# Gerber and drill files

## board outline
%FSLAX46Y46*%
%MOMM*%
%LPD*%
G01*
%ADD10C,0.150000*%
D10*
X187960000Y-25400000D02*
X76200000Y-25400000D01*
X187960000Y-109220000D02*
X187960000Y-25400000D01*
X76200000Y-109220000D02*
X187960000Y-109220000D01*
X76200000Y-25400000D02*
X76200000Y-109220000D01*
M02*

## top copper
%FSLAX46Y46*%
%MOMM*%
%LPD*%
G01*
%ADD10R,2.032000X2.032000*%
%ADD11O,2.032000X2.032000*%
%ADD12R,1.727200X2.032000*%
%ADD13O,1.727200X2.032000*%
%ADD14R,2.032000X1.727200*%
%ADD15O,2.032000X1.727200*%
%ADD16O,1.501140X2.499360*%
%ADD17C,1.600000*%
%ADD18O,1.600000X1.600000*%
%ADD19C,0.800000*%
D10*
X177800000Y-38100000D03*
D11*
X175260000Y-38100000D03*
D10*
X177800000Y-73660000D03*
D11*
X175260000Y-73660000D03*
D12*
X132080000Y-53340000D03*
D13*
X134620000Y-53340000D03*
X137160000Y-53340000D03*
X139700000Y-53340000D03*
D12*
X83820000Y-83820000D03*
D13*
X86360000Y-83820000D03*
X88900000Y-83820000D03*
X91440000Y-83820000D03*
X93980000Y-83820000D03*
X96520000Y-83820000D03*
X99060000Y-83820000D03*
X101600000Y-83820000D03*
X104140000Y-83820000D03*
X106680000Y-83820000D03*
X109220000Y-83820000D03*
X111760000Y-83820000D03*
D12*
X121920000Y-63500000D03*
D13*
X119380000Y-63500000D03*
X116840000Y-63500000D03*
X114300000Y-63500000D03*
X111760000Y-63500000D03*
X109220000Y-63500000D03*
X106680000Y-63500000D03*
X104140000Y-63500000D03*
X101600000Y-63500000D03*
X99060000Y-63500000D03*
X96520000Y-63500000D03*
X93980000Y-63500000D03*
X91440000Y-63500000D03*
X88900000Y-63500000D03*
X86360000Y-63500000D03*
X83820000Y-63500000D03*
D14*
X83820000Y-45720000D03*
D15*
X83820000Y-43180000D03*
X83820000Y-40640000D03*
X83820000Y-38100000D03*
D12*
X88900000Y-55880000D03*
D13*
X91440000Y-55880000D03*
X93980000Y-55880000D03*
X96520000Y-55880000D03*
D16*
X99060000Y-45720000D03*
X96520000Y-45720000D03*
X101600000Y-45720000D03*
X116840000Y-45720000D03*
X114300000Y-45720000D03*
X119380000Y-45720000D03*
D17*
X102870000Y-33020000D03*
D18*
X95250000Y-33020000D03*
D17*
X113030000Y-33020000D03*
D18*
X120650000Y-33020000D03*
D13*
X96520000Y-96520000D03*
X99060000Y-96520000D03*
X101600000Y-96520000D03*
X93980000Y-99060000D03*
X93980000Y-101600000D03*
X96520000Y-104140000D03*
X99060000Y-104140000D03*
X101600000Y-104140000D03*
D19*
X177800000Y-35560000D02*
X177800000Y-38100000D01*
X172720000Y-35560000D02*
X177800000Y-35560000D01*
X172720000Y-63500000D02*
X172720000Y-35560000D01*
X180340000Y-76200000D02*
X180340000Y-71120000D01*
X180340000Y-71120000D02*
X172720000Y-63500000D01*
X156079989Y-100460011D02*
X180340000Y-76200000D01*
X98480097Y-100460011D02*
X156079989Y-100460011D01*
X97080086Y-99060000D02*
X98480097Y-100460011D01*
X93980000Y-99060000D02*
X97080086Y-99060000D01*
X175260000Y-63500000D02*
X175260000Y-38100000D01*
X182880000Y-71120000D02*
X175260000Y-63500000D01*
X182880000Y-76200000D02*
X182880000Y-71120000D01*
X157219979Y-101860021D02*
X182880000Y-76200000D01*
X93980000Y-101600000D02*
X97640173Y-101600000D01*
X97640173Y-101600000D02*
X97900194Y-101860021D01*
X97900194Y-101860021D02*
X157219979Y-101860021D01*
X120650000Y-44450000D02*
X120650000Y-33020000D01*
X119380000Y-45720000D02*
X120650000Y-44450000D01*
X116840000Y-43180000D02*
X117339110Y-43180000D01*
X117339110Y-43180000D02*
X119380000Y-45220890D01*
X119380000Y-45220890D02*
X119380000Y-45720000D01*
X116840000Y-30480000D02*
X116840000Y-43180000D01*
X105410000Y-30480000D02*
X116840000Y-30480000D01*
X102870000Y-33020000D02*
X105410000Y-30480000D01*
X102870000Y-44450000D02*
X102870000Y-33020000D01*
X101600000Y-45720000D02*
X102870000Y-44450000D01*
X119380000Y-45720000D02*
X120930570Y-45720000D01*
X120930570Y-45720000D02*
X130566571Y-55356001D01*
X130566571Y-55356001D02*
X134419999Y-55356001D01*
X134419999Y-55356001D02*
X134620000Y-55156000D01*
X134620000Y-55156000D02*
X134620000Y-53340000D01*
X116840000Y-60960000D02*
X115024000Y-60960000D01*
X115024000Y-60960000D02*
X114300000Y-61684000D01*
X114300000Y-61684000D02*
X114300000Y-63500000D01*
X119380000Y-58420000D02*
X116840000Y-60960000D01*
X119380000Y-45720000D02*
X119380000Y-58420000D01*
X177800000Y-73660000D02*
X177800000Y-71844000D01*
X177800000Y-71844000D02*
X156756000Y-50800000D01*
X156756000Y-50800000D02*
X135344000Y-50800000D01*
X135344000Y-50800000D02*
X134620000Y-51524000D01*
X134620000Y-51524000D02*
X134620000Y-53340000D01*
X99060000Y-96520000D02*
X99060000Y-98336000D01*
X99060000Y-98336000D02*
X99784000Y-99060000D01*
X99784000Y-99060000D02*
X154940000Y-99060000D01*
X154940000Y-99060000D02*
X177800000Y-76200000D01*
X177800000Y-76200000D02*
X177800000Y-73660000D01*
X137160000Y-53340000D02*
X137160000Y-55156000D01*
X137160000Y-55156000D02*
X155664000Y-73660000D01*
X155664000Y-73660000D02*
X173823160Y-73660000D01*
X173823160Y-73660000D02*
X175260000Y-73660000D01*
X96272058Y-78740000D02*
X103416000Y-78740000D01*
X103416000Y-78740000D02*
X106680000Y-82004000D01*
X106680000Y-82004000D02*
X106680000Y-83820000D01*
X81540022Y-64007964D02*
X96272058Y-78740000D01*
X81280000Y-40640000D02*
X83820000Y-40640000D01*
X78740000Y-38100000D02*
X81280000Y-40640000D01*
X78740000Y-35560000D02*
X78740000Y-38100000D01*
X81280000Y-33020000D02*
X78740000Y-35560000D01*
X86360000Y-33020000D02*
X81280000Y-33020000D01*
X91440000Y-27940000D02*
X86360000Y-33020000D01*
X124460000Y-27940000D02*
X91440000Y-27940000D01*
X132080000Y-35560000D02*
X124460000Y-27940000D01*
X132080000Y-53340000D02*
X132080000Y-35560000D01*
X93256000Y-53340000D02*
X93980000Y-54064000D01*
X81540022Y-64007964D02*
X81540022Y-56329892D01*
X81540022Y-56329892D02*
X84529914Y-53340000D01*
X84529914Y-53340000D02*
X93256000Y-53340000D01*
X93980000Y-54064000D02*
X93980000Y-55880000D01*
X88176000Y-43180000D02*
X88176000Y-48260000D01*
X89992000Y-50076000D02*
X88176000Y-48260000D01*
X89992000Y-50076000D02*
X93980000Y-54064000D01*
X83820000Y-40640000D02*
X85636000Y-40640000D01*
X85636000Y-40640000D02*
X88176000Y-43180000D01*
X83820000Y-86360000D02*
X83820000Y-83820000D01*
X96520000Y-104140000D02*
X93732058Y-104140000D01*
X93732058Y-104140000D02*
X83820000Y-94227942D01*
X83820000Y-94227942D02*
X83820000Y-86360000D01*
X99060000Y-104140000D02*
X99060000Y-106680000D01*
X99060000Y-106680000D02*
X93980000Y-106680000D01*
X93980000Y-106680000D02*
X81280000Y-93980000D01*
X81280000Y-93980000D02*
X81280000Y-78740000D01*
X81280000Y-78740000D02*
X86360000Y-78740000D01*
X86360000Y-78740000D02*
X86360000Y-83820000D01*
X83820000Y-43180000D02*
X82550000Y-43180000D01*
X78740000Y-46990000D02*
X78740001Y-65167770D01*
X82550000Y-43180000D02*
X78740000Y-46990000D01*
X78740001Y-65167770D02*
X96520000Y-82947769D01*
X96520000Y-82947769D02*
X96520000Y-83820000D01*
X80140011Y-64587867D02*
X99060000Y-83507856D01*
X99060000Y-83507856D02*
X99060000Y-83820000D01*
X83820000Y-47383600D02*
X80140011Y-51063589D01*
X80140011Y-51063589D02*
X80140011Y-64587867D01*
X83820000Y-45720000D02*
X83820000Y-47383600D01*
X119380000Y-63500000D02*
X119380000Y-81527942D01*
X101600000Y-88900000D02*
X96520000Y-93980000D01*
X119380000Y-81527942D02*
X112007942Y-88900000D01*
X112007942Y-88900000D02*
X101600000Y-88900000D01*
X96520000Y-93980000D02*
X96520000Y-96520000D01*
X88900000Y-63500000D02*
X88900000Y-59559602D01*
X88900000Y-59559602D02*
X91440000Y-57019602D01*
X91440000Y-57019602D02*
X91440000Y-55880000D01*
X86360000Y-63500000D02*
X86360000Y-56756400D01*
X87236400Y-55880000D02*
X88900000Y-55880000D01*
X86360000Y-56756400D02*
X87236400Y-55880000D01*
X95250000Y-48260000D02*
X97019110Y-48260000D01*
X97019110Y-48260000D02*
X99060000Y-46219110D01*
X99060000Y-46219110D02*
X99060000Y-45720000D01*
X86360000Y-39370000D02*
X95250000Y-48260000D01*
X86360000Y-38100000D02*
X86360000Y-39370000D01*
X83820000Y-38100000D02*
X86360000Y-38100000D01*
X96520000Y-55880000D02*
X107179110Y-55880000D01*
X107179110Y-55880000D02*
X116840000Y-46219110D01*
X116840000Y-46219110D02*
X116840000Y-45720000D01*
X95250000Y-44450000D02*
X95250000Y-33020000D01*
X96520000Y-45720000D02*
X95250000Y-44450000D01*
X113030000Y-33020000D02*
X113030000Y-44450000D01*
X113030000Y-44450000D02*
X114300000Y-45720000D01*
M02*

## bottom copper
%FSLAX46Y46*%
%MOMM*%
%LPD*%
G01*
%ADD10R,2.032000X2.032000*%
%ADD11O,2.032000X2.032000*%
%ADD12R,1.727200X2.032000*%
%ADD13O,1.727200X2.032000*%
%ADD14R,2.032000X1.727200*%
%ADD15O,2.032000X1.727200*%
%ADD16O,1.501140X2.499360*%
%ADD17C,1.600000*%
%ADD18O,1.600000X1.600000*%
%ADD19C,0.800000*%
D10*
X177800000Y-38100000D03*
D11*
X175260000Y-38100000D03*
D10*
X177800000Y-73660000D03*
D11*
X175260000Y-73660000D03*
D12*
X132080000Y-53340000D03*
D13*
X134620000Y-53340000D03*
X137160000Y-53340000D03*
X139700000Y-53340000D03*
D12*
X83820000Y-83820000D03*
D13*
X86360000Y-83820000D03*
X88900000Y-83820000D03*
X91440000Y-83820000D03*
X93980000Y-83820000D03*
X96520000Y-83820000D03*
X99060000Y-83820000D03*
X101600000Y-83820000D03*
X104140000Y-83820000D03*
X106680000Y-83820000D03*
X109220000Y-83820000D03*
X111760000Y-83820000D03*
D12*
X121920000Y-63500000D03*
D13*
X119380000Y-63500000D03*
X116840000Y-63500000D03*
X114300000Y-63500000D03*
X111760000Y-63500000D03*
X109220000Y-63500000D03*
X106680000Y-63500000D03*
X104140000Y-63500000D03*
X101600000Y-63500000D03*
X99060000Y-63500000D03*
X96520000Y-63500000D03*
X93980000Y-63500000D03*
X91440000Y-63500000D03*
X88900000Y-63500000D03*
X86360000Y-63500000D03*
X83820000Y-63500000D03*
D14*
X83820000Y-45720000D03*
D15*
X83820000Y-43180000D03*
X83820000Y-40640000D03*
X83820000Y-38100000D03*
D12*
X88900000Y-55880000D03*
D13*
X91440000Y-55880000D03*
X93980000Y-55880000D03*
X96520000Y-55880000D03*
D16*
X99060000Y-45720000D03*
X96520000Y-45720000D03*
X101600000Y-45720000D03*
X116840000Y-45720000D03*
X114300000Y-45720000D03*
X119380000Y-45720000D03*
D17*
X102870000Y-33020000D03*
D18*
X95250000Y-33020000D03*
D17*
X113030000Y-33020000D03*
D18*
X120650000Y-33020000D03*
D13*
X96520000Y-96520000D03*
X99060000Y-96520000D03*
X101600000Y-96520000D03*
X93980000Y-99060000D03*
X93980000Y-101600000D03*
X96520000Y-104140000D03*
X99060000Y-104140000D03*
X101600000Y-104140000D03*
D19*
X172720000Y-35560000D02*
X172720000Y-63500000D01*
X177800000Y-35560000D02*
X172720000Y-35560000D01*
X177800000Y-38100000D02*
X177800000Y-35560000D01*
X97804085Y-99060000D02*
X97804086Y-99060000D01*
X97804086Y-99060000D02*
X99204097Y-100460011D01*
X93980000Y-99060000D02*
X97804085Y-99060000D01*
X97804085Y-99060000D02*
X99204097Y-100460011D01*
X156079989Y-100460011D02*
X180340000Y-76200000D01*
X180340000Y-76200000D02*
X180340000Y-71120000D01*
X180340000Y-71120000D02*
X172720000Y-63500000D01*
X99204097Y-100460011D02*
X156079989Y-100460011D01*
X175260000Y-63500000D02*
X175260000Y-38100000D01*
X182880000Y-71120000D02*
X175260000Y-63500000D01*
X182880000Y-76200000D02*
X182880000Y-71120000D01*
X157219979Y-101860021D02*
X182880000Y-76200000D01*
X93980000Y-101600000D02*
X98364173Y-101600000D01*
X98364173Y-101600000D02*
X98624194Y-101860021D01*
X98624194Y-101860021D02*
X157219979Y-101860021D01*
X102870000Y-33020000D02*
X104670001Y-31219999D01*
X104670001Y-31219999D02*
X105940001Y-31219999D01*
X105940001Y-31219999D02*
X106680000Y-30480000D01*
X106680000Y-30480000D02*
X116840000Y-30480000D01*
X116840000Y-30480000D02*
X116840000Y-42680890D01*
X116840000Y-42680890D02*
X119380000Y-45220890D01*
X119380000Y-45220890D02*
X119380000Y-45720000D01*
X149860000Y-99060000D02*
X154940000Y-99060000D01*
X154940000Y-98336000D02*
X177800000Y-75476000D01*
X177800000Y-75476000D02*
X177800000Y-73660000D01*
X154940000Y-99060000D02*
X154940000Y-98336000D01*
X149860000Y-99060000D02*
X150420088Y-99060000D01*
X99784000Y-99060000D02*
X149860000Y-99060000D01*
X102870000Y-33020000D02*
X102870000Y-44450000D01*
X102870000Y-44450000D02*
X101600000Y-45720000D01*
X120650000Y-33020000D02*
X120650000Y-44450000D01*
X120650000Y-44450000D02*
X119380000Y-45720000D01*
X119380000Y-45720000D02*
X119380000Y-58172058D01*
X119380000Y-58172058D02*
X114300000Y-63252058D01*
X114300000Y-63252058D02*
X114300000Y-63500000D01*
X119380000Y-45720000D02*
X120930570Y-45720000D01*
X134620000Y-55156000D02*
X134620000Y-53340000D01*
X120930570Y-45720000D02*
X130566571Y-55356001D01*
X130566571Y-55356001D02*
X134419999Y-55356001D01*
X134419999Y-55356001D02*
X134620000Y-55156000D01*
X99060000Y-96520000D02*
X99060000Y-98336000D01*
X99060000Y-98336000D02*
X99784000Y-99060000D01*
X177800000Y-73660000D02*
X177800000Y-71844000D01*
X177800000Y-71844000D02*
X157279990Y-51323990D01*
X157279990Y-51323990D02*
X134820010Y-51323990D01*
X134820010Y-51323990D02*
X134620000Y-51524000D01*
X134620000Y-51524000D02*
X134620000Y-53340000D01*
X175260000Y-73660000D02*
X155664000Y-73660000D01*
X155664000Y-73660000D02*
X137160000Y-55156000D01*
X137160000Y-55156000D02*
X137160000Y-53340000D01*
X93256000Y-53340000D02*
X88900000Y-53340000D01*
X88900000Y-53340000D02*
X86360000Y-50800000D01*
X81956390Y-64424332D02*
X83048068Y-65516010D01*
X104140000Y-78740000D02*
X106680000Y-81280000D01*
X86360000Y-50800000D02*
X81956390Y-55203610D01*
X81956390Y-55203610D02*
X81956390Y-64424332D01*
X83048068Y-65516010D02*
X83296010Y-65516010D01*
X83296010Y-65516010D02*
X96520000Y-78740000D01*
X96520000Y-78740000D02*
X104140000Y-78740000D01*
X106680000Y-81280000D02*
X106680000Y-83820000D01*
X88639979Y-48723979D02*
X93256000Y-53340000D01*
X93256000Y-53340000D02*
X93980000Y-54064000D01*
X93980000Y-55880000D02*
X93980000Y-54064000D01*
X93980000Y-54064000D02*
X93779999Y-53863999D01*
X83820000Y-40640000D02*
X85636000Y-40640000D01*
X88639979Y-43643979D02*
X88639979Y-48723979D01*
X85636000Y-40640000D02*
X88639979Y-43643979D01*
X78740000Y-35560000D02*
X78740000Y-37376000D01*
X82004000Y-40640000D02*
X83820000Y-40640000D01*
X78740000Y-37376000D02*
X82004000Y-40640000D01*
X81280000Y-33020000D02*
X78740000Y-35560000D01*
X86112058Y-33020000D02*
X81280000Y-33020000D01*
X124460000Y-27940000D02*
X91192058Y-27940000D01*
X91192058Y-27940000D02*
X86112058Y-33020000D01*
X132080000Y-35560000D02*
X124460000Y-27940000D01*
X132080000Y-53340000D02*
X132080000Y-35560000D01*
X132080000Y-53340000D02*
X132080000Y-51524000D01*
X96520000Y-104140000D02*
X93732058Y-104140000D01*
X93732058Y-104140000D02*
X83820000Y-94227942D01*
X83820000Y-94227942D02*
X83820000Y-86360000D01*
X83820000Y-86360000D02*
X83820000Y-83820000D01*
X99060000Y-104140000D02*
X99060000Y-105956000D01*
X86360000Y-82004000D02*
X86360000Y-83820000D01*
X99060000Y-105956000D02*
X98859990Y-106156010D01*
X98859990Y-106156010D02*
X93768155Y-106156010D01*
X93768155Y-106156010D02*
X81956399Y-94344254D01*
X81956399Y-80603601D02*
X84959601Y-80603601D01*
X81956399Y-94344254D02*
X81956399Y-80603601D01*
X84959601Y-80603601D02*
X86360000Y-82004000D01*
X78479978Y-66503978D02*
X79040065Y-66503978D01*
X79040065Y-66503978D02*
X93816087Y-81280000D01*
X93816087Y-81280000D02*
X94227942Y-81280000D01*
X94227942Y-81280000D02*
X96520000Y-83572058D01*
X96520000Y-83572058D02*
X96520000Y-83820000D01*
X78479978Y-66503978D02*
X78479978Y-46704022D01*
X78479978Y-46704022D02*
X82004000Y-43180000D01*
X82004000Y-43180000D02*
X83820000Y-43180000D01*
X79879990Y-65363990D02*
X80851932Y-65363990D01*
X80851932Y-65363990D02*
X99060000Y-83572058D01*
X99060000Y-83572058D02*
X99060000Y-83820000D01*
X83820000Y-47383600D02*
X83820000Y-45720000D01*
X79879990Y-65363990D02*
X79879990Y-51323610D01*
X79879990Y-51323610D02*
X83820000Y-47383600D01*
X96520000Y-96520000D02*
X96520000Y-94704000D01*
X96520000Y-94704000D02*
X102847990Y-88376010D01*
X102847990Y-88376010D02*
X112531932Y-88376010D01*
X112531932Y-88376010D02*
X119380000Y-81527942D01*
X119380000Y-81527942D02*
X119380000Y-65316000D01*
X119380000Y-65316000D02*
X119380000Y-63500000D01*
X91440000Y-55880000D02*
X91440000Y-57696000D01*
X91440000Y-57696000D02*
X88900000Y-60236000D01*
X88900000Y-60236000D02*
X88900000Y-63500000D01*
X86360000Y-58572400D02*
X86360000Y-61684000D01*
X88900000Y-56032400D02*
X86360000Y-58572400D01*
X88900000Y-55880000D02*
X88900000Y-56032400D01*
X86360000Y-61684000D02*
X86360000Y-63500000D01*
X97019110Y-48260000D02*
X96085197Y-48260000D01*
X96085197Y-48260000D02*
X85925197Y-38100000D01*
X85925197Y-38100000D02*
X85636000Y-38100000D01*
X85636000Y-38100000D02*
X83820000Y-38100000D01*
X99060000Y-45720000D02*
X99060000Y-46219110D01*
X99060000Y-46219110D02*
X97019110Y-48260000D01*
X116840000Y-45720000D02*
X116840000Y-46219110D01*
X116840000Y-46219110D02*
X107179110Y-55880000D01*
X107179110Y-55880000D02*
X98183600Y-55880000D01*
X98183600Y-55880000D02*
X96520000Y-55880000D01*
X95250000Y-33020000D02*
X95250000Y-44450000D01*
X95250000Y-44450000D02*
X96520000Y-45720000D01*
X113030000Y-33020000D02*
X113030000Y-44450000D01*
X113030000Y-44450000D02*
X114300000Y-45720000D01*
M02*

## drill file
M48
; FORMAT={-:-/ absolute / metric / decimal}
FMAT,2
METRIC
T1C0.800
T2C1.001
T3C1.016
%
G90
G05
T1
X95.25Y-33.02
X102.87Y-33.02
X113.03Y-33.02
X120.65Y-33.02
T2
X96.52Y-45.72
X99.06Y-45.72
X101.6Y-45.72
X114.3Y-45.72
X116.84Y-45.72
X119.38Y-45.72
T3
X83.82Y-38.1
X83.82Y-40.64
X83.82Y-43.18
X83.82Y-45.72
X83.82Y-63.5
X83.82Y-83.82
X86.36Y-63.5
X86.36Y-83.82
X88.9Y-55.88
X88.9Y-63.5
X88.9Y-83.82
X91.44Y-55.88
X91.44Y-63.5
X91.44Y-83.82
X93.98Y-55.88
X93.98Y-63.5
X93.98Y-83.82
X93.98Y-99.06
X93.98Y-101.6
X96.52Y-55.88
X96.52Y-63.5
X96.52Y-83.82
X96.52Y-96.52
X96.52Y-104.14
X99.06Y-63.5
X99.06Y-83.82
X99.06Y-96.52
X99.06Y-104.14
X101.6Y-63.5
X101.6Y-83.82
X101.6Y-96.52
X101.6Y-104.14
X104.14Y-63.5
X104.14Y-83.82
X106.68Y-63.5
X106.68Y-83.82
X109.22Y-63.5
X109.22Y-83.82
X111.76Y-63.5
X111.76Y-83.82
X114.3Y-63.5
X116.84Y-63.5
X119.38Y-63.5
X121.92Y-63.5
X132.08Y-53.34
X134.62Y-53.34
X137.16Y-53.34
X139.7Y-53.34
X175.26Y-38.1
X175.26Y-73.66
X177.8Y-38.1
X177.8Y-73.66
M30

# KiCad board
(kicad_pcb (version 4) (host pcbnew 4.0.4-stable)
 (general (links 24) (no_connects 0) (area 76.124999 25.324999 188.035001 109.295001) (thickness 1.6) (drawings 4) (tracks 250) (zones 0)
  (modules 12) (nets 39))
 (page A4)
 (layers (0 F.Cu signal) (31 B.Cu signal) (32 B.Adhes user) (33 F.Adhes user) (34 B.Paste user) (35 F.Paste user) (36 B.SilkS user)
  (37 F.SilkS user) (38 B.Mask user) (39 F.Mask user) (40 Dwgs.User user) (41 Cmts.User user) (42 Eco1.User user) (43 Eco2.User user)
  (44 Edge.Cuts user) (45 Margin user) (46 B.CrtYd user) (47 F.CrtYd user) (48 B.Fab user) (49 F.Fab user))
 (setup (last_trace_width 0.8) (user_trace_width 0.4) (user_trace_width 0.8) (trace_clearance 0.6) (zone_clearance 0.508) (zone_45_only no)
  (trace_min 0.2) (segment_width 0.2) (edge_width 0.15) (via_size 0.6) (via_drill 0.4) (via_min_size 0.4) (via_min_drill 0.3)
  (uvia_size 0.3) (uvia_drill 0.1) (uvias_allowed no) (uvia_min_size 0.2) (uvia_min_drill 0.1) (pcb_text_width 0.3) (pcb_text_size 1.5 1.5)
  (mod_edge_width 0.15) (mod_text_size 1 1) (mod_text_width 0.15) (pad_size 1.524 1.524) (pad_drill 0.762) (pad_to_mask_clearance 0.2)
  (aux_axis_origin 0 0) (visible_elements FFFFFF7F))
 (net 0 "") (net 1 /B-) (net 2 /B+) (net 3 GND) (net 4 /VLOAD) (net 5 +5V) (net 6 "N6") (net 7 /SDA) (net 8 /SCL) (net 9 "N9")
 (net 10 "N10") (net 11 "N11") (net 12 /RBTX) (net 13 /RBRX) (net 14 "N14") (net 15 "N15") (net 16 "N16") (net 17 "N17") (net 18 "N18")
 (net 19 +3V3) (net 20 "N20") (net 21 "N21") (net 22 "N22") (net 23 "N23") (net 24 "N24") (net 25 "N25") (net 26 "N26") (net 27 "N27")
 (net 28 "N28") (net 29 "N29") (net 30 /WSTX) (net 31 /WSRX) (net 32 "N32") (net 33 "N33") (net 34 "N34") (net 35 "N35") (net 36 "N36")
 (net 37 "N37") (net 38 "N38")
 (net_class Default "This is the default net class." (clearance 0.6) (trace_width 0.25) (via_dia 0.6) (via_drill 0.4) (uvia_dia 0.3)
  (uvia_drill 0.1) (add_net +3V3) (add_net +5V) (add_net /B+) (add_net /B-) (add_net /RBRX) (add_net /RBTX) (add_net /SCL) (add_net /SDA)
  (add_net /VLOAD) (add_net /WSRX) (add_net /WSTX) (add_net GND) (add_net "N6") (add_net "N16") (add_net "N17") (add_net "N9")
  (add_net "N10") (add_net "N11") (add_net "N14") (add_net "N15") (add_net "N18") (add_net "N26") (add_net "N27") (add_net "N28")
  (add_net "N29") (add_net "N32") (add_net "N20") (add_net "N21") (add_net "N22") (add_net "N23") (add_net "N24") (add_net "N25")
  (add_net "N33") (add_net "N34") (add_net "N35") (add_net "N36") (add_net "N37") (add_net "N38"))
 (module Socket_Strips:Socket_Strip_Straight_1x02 (layer F.Cu) (at 177.8 38.1 180)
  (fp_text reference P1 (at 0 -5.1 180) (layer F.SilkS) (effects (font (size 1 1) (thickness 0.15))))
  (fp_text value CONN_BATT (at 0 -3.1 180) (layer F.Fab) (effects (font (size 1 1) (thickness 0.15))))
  (pad 1 thru_hole rect (at 0 0 180) (size 2.032 2.032) (drill 1.016) (layers *.Cu *.Mask) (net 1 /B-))
  (pad 2 thru_hole oval (at 2.54 0 180) (size 2.032 2.032) (drill 1.016) (layers *.Cu *.Mask) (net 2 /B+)))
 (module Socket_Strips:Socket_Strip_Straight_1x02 (layer F.Cu) (at 177.8 73.66 180)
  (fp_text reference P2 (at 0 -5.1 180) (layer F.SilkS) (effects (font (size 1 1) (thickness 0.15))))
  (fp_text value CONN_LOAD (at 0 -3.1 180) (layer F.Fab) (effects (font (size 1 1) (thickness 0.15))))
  (pad 1 thru_hole rect (at 0 0 180) (size 2.032 2.032) (drill 1.016) (layers *.Cu *.Mask) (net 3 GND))
  (pad 2 thru_hole oval (at 2.54 0 180) (size 2.032 2.032) (drill 1.016) (layers *.Cu *.Mask) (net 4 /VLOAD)))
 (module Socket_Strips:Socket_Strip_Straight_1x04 (layer F.Cu) (at 132.08 53.34)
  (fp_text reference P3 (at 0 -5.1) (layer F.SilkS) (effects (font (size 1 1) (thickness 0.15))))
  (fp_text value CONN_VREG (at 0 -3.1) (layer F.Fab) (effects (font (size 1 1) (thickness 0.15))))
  (pad 1 thru_hole rect (at 0 0) (size 1.7272 2.032) (drill 1.016) (layers *.Cu *.Mask) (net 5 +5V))
  (pad 2 thru_hole oval (at 2.54 0) (size 1.7272 2.032) (drill 1.016) (layers *.Cu *.Mask) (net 3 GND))
  (pad 3 thru_hole oval (at 5.08 0) (size 1.7272 2.032) (drill 1.016) (layers *.Cu *.Mask) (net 4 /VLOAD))
  (pad 4 thru_hole oval (at 7.62 0) (size 1.7272 2.032) (drill 1.016) (layers *.Cu *.Mask) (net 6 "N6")))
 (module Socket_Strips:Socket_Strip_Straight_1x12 (layer F.Cu) (at 83.82 83.82)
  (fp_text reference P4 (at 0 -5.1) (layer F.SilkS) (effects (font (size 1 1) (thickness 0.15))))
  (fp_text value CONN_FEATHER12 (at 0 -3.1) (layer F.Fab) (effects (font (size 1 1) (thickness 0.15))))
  (pad 1 thru_hole rect (at 0 0) (size 1.7272 2.032) (drill 1.016) (layers *.Cu *.Mask) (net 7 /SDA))
  (pad 2 thru_hole oval (at 2.54 0) (size 1.7272 2.032) (drill 1.016) (layers *.Cu *.Mask) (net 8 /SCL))
  (pad 3 thru_hole oval (at 5.08 0) (size 1.7272 2.032) (drill 1.016) (layers *.Cu *.Mask) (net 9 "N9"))
  (pad 4 thru_hole oval (at 7.62 0) (size 1.7272 2.032) (drill 1.016) (layers *.Cu *.Mask) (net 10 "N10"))
  (pad 5 thru_hole oval (at 10.16 0) (size 1.7272 2.032) (drill 1.016) (layers *.Cu *.Mask) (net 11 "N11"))
  (pad 6 thru_hole oval (at 12.7 0) (size 1.7272 2.032) (drill 1.016) (layers *.Cu *.Mask) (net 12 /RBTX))
  (pad 7 thru_hole oval (at 15.24 0) (size 1.7272 2.032) (drill 1.016) (layers *.Cu *.Mask) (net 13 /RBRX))
  (pad 8 thru_hole oval (at 17.78 0) (size 1.7272 2.032) (drill 1.016) (layers *.Cu *.Mask) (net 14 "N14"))
  (pad 9 thru_hole oval (at 20.32 0) (size 1.7272 2.032) (drill 1.016) (layers *.Cu *.Mask) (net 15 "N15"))
  (pad 10 thru_hole oval (at 22.86 0) (size 1.7272 2.032) (drill 1.016) (layers *.Cu *.Mask) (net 5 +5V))
  (pad 11 thru_hole oval (at 25.4 0) (size 1.7272 2.032) (drill 1.016) (layers *.Cu *.Mask) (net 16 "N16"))
  (pad 12 thru_hole oval (at 27.94 0) (size 1.7272 2.032) (drill 1.016) (layers *.Cu *.Mask) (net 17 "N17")))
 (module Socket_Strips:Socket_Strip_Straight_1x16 (layer F.Cu) (at 121.92 63.5 180)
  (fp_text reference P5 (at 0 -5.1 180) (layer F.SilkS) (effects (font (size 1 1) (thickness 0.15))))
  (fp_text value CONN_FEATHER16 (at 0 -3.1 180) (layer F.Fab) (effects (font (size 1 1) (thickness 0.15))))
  (pad 1 thru_hole rect (at 0 0 180) (size 1.7272 2.032) (drill 1.016) (layers *.Cu *.Mask) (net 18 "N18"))
  (pad 2 thru_hole oval (at 2.54 0 180) (size 1.7272 2.032) (drill 1.016) (layers *.Cu *.Mask) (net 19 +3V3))
  (pad 3 thru_hole oval (at 5.08 0 180) (size 1.7272 2.032) (drill 1.016) (layers *.Cu *.Mask) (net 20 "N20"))
  (pad 4 thru_hole oval (at 7.62 0 180) (size 1.7272 2.032) (drill 1.016) (layers *.Cu *.Mask) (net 3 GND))
  (pad 5 thru_hole oval (at 10.16 0 180) (size 1.7272 2.032) (drill 1.016) (layers *.Cu *.Mask) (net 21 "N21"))
  (pad 6 thru_hole oval (at 12.7 0 180) (size 1.7272 2.032) (drill 1.016) (layers *.Cu *.Mask) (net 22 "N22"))
  (pad 7 thru_hole oval (at 15.24 0 180) (size 1.7272 2.032) (drill 1.016) (layers *.Cu *.Mask) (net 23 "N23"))
  (pad 8 thru_hole oval (at 17.78 0 180) (size 1.7272 2.032) (drill 1.016) (layers *.Cu *.Mask) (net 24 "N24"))
  (pad 9 thru_hole oval (at 20.32 0 180) (size 1.7272 2.032) (drill 1.016) (layers *.Cu *.Mask) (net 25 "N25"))
  (pad 10 thru_hole oval (at 22.86 0 180) (size 1.7272 2.032) (drill 1.016) (layers *.Cu *.Mask) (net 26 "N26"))
  (pad 11 thru_hole oval (at 25.4 0 180) (size 1.7272 2.032) (drill 1.016) (layers *.Cu *.Mask) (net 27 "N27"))
  (pad 12 thru_hole oval (at 27.94 0 180) (size 1.7272 2.032) (drill 1.016) (layers *.Cu *.Mask) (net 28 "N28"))
  (pad 13 thru_hole oval (at 30.48 0 180) (size 1.7272 2.032) (drill 1.016) (layers *.Cu *.Mask) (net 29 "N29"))
  (pad 14 thru_hole oval (at 33.02 0 180) (size 1.7272 2.032) (drill 1.016) (layers *.Cu *.Mask) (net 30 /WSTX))
  (pad 15 thru_hole oval (at 35.56 0 180) (size 1.7272 2.032) (drill 1.016) (layers *.Cu *.Mask) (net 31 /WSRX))
  (pad 16 thru_hole oval (at 38.1 0 180) (size 1.7272 2.032) (drill 1.016) (layers *.Cu *.Mask) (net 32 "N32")))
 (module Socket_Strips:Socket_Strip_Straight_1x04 (layer F.Cu) (at 83.82 45.72 90)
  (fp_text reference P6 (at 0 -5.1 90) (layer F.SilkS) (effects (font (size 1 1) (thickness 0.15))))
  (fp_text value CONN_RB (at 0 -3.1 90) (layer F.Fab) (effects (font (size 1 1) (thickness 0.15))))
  (pad 1 thru_hole rect (at 0 0 90) (size 1.7272 2.032) (drill 1.016) (layers *.Cu *.Mask) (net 13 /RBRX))
  (pad 2 thru_hole oval (at 2.54 0 90) (size 1.7272 2.032) (drill 1.016) (layers *.Cu *.Mask) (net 12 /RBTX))
  (pad 3 thru_hole oval (at 5.08 0 90) (size 1.7272 2.032) (drill 1.016) (layers *.Cu *.Mask) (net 5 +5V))
  (pad 4 thru_hole oval (at 7.62 0 90) (size 1.7272 2.032) (drill 1.016) (layers *.Cu *.Mask) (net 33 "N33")))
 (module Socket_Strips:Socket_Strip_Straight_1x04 (layer F.Cu) (at 88.9 55.88)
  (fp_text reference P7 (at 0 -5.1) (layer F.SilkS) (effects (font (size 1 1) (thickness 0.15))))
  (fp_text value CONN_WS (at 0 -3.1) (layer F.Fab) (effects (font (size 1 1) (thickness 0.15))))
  (pad 1 thru_hole rect (at 0 0) (size 1.7272 2.032) (drill 1.016) (layers *.Cu *.Mask) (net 31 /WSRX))
  (pad 2 thru_hole oval (at 2.54 0) (size 1.7272 2.032) (drill 1.016) (layers *.Cu *.Mask) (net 30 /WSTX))
  (pad 3 thru_hole oval (at 5.08 0) (size 1.7272 2.032) (drill 1.016) (layers *.Cu *.Mask) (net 5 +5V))
  (pad 4 thru_hole oval (at 7.62 0) (size 1.7272 2.032) (drill 1.016) (layers *.Cu *.Mask) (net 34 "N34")))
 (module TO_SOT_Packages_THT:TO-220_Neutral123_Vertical (layer F.Cu) (at 99.06 45.72)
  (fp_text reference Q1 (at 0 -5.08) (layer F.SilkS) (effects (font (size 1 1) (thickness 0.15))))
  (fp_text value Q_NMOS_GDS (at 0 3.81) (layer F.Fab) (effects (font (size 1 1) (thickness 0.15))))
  (pad 2 thru_hole oval (at 0 0 90) (size 2.49936 1.50114) (drill 1.00076) (layers *.Cu *.Mask) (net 33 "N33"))
  (pad 1 thru_hole oval (at -2.54 0 90) (size 2.49936 1.50114) (drill 1.00076) (layers *.Cu *.Mask) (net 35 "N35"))
  (pad 3 thru_hole oval (at 2.54 0 90) (size 2.49936 1.50114) (drill 1.00076) (layers *.Cu *.Mask) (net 3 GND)))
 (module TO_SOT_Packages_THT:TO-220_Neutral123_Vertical (layer F.Cu) (at 116.84 45.72)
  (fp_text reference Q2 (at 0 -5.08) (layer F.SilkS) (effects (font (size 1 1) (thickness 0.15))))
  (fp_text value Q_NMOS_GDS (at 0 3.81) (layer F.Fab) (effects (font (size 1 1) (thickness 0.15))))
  (pad 2 thru_hole oval (at 0 0 90) (size 2.49936 1.50114) (drill 1.00076) (layers *.Cu *.Mask) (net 34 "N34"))
  (pad 1 thru_hole oval (at -2.54 0 90) (size 2.49936 1.50114) (drill 1.00076) (layers *.Cu *.Mask) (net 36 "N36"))
  (pad 3 thru_hole oval (at 2.54 0 90) (size 2.49936 1.50114) (drill 1.00076) (layers *.Cu *.Mask) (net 3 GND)))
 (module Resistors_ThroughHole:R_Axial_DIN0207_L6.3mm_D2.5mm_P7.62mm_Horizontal (layer F.Cu) (at 102.87 33.02 180)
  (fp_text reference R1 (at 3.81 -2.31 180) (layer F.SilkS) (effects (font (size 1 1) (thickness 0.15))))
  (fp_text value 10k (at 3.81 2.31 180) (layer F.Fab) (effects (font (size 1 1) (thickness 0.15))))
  (pad 1 thru_hole circle (at 0 0 180) (size 1.6 1.6) (drill 0.8) (layers *.Cu *.Mask) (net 3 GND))
  (pad 2 thru_hole oval (at 7.62 0 180) (size 1.6 1.6) (drill 0.8) (layers *.Cu *.Mask) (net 35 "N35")))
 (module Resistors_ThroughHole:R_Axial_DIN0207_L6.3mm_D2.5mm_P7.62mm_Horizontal (layer F.Cu) (at 113.03 33.02)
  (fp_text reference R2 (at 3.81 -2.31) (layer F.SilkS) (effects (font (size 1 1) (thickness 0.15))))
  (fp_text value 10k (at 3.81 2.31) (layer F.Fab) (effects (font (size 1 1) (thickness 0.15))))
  (pad 1 thru_hole circle (at 0 0) (size 1.6 1.6) (drill 0.8) (layers *.Cu *.Mask) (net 36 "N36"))
  (pad 2 thru_hole oval (at 7.62 0) (size 1.6 1.6) (drill 0.8) (layers *.Cu *.Mask) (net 3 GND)))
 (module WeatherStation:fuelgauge (layer F.Cu) (at 93.98 96.52)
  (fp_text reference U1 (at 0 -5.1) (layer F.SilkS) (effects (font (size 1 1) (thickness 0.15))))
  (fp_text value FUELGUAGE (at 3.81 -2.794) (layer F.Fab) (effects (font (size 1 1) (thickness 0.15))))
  (pad 3 thru_hole oval (at 2.54 0) (size 1.7272 2.032) (drill 1.016) (layers *.Cu *.Mask) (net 19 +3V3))
  (pad 4 thru_hole oval (at 5.08 0) (size 1.7272 2.032) (drill 1.016) (layers *.Cu *.Mask) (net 3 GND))
  (pad 5 thru_hole oval (at 7.62 0) (size 1.7272 2.032) (drill 1.016) (layers *.Cu *.Mask) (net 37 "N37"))
  (pad 2 thru_hole oval (at 0 2.54) (size 1.7272 2.032) (drill 1.016) (layers *.Cu *.Mask) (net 1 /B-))
  (pad 1 thru_hole oval (at 0 5.08) (size 1.7272 2.032) (drill 1.016) (layers *.Cu *.Mask) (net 2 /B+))
  (pad 8 thru_hole oval (at 2.54 7.62) (size 1.7272 2.032) (drill 1.016) (layers *.Cu *.Mask) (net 7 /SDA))
  (pad 7 thru_hole oval (at 5.08 7.62) (size 1.7272 2.032) (drill 1.016) (layers *.Cu *.Mask) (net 8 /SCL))
  (pad 6 thru_hole oval (at 7.62 7.62) (size 1.7272 2.032) (drill 1.016) (layers *.Cu *.Mask) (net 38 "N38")))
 (gr_line (start 187.96 25.4) (end 76.2 25.4) (angle 90) (layer Edge.Cuts) (width 0.15))
 (gr_line (start 187.96 109.22) (end 187.96 25.4) (angle 90) (layer Edge.Cuts) (width 0.15))
 (gr_line (start 76.2 109.22) (end 187.96 109.22) (angle 90) (layer Edge.Cuts) (width 0.15))
 (gr_line (start 76.2 25.4) (end 76.2 109.22) (angle 90) (layer Edge.Cuts) (width 0.15))
 (segment (start 172.72 35.56) (end 172.72 63.5) (width 0.8) (layer B.Cu) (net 1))
 (segment (start 177.8 35.56) (end 172.72 35.56) (width 0.8) (layer B.Cu) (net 1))
 (segment (start 177.8 38.1) (end 177.8 35.56) (width 0.8) (layer B.Cu) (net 1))
 (segment (start 177.8 35.56) (end 177.8 38.1) (width 0.8) (layer F.Cu) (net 1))
 (segment (start 172.72 35.56) (end 177.8 35.56) (width 0.8) (layer F.Cu) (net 1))
 (segment (start 172.72 63.5) (end 172.72 35.56) (width 0.8) (layer F.Cu) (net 1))
 (segment (start 180.34 76.2) (end 180.34 71.12) (width 0.8) (layer F.Cu) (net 1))
 (segment (start 180.34 71.12) (end 172.72 63.5) (width 0.8) (layer F.Cu) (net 1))
 (segment (start 156.079989 100.460011) (end 180.34 76.2) (width 0.8) (layer F.Cu) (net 1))
 (segment (start 98.480097 100.460011) (end 156.079989 100.460011) (width 0.8) (layer F.Cu) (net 1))
 (segment (start 97.080086 99.06) (end 98.480097 100.460011) (width 0.8) (layer F.Cu) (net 1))
 (segment (start 93.98 99.06) (end 97.080086 99.06) (width 0.8) (layer F.Cu) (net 1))
 (segment (start 97.804085 99.06) (end 97.804086 99.06) (width 0.8) (layer B.Cu) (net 1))
 (segment (start 97.804086 99.06) (end 99.204097 100.460011) (width 0.8) (layer B.Cu) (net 1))
 (segment (start 93.98 99.06) (end 97.804085 99.06) (width 0.8) (layer B.Cu) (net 1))
 (segment (start 97.804085 99.06) (end 99.204097 100.460011) (width 0.8) (layer B.Cu) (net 1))
 (segment (start 156.079989 100.460011) (end 180.34 76.2) (width 0.8) (layer B.Cu) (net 1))
 (segment (start 180.34 76.2) (end 180.34 71.12) (width 0.8) (layer B.Cu) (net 1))
 (segment (start 180.34 71.12) (end 172.72 63.5) (width 0.8) (layer B.Cu) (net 1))
 (segment (start 99.204097 100.460011) (end 156.079989 100.460011) (width 0.8) (layer B.Cu) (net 1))
 (segment (start 175.26 63.5) (end 175.26 38.1) (width 0.8) (layer B.Cu) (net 2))
 (segment (start 182.88 71.12) (end 175.26 63.5) (width 0.8) (layer B.Cu) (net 2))
 (segment (start 182.88 76.2) (end 182.88 71.12) (width 0.8) (layer B.Cu) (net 2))
 (segment (start 157.219979 101.860021) (end 182.88 76.2) (width 0.8) (layer B.Cu) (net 2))
 (segment (start 93.98 101.6) (end 98.364173 101.6) (width 0.8) (layer B.Cu) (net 2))
 (segment (start 98.364173 101.6) (end 98.624194 101.860021) (width 0.8) (layer B.Cu) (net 2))
 (segment (start 98.624194 101.860021) (end 157.219979 101.860021) (width 0.8) (layer B.Cu) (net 2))
 (segment (start 175.26 63.5) (end 175.26 38.1) (width 0.8) (layer F.Cu) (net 2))
 (segment (start 182.88 71.12) (end 175.26 63.5) (width 0.8) (layer F.Cu) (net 2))
 (segment (start 182.88 76.2) (end 182.88 71.12) (width 0.8) (layer F.Cu) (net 2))
 (segment (start 157.219979 101.860021) (end 182.88 76.2) (width 0.8) (layer F.Cu) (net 2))
 (segment (start 93.98 101.6) (end 97.640173 101.6) (width 0.8) (layer F.Cu) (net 2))
 (segment (start 97.640173 101.6) (end 97.900194 101.860021) (width 0.8) (layer F.Cu) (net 2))
 (segment (start 97.900194 101.860021) (end 157.219979 101.860021) (width 0.8) (layer F.Cu) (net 2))
 (segment (start 120.65 44.45) (end 120.65 33.02) (width 0.8) (layer F.Cu) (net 3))
 (segment (start 119.38 45.72) (end 120.65 44.45) (width 0.8) (layer F.Cu) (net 3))
 (segment (start 116.84 43.18) (end 117.33911 43.18) (width 0.8) (layer F.Cu) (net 3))
 (segment (start 117.33911 43.18) (end 119.38 45.22089) (width 0.8) (layer F.Cu) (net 3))
 (segment (start 119.38 45.22089) (end 119.38 45.72) (width 0.8) (layer F.Cu) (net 3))
 (segment (start 116.84 30.48) (end 116.84 43.18) (width 0.8) (layer F.Cu) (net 3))
 (segment (start 105.41 30.48) (end 116.84 30.48) (width 0.8) (layer F.Cu) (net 3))
 (segment (start 102.87 33.02) (end 105.41 30.48) (width 0.8) (layer F.Cu) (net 3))
 (segment (start 102.87 44.45) (end 102.87 33.02) (width 0.8) (layer F.Cu) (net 3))
 (segment (start 101.6 45.72) (end 102.87 44.45) (width 0.8) (layer F.Cu) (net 3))
 (segment (start 119.38 45.72) (end 120.93057 45.72) (width 0.8) (layer F.Cu) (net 3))
 (segment (start 120.93057 45.72) (end 130.566571 55.356001) (width 0.8) (layer F.Cu) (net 3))
 (segment (start 130.566571 55.356001) (end 134.419999 55.356001) (width 0.8) (layer F.Cu) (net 3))
 (segment (start 134.419999 55.356001) (end 134.62 55.156) (width 0.8) (layer F.Cu) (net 3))
 (segment (start 134.62 55.156) (end 134.62 53.34) (width 0.8) (layer F.Cu) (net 3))
 (segment (start 116.84 60.96) (end 115.024 60.96) (width 0.8) (layer F.Cu) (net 3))
 (segment (start 115.024 60.96) (end 114.3 61.684) (width 0.8) (layer F.Cu) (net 3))
 (segment (start 114.3 61.684) (end 114.3 63.5) (width 0.8) (layer F.Cu) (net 3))
 (segment (start 119.38 58.42) (end 116.84 60.96) (width 0.8) (layer F.Cu) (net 3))
 (segment (start 119.38 45.72) (end 119.38 58.42) (width 0.8) (layer F.Cu) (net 3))
 (segment (start 177.8 73.66) (end 177.8 71.844) (width 0.8) (layer F.Cu) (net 3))
 (segment (start 177.8 71.844) (end 156.756 50.8) (width 0.8) (layer F.Cu) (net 3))
 (segment (start 156.756 50.8) (end 135.344 50.8) (width 0.8) (layer F.Cu) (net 3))
 (segment (start 135.344 50.8) (end 134.62 51.524) (width 0.8) (layer F.Cu) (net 3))
 (segment (start 134.62 51.524) (end 134.62 53.34) (width 0.8) (layer F.Cu) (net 3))
 (segment (start 99.06 96.52) (end 99.06 98.336) (width 0.8) (layer F.Cu) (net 3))
 (segment (start 99.06 98.336) (end 99.784 99.06) (width 0.8) (layer F.Cu) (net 3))
 (segment (start 99.784 99.06) (end 154.94 99.06) (width 0.8) (layer F.Cu) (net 3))
 (segment (start 154.94 99.06) (end 177.8 76.2) (width 0.8) (layer F.Cu) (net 3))
 (segment (start 177.8 76.2) (end 177.8 73.66) (width 0.8) (layer F.Cu) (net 3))
 (segment (start 102.87 33.02) (end 104.670001 31.219999) (width 0.8) (layer B.Cu) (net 3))
 (segment (start 104.670001 31.219999) (end 105.940001 31.219999) (width 0.8) (layer B.Cu) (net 3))
 (segment (start 105.940001 31.219999) (end 106.68 30.48) (width 0.8) (layer B.Cu) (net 3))
 (segment (start 106.68 30.48) (end 116.84 30.48) (width 0.8) (layer B.Cu) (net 3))
 (segment (start 116.84 30.48) (end 116.84 42.68089) (width 0.8) (layer B.Cu) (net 3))
 (segment (start 116.84 42.68089) (end 119.38 45.22089) (width 0.8) (layer B.Cu) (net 3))
 (segment (start 119.38 45.22089) (end 119.38 45.72) (width 0.8) (layer B.Cu) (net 3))
 (segment (start 149.86 99.06) (end 154.94 99.06) (width 0.8) (layer B.Cu) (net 3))
 (segment (start 154.94 98.336) (end 177.8 75.476) (width 0.8) (layer B.Cu) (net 3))
 (segment (start 177.8 75.476) (end 177.8 73.66) (width 0.8) (layer B.Cu) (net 3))
 (segment (start 154.94 99.06) (end 154.94 98.336) (width 0.8) (layer B.Cu) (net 3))
 (segment (start 149.86 99.06) (end 150.420088 99.06) (width 0.8) (layer B.Cu) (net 3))
 (segment (start 99.784 99.06) (end 149.86 99.06) (width 0.8) (layer B.Cu) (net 3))
 (segment (start 102.87 33.02) (end 102.87 44.45) (width 0.8) (layer B.Cu) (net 3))
 (segment (start 102.87 44.45) (end 101.6 45.72) (width 0.8) (layer B.Cu) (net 3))
 (segment (start 120.65 33.02) (end 120.65 44.45) (width 0.8) (layer B.Cu) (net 3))
 (segment (start 120.65 44.45) (end 119.38 45.72) (width 0.8) (layer B.Cu) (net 3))
 (segment (start 119.38 45.72) (end 119.38 58.172058) (width 0.8) (layer B.Cu) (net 3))
 (segment (start 119.38 58.172058) (end 114.3 63.252058) (width 0.8) (layer B.Cu) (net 3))
 (segment (start 114.3 63.252058) (end 114.3 63.5) (width 0.8) (layer B.Cu) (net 3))
 (segment (start 119.38 45.72) (end 120.93057 45.72) (width 0.8) (layer B.Cu) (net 3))
 (segment (start 134.62 55.156) (end 134.62 53.34) (width 0.8) (layer B.Cu) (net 3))
 (segment (start 120.93057 45.72) (end 130.566571 55.356001) (width 0.8) (layer B.Cu) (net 3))
 (segment (start 130.566571 55.356001) (end 134.419999 55.356001) (width 0.8) (layer B.Cu) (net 3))
 (segment (start 134.419999 55.356001) (end 134.62 55.156) (width 0.8) (layer B.Cu) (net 3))
 (segment (start 99.06 96.52) (end 99.06 98.336) (width 0.8) (layer B.Cu) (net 3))
 (segment (start 99.06 98.336) (end 99.784 99.06) (width 0.8) (layer B.Cu) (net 3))
 (segment (start 177.8 73.66) (end 177.8 71.844) (width 0.8) (layer B.Cu) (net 3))
 (segment (start 177.8 71.844) (end 157.27999 51.32399) (width 0.8) (layer B.Cu) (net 3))
 (segment (start 157.27999 51.32399) (end 134.82001 51.32399) (width 0.8) (layer B.Cu) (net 3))
 (segment (start 134.82001 51.32399) (end 134.62 51.524) (width 0.8) (layer B.Cu) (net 3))
 (segment (start 134.62 51.524) (end 134.62 53.34) (width 0.8) (layer B.Cu) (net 3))
 (segment (start 137.16 53.34) (end 137.16 55.156) (width 0.8) (layer F.Cu) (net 4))
 (segment (start 137.16 55.156) (end 155.664 73.66) (width 0.8) (layer F.Cu) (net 4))
 (segment (start 155.664 73.66) (end 173.82316 73.66) (width 0.8) (layer F.Cu) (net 4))
 (segment (start 173.82316 73.66) (end 175.26 73.66) (width 0.8) (layer F.Cu) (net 4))
 (segment (start 175.26 73.66) (end 155.664 73.66) (width 0.8) (layer B.Cu) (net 4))
 (segment (start 155.664 73.66) (end 137.16 55.156) (width 0.8) (layer B.Cu) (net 4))
 (segment (start 137.16 55.156) (end 137.16 53.34) (width 0.8) (layer B.Cu) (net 4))
 (segment (start 93.256 53.34) (end 88.9 53.34) (width 0.8) (layer B.Cu) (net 5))
 (segment (start 88.9 53.34) (end 86.36 50.8) (width 0.8) (layer B.Cu) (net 5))
 (segment (start 81.95639 64.424332) (end 83.048068 65.51601) (width 0.8) (layer B.Cu) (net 5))
 (segment (start 104.14 78.74) (end 106.68 81.28) (width 0.8) (layer B.Cu) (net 5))
 (segment (start 86.36 50.8) (end 81.95639 55.20361) (width 0.8) (layer B.Cu) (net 5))
 (segment (start 81.95639 55.20361) (end 81.95639 64.424332) (width 0.8) (layer B.Cu) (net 5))
 (segment (start 83.048068 65.51601) (end 83.29601 65.51601) (width 0.8) (layer B.Cu) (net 5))
 (segment (start 83.29601 65.51601) (end 96.52 78.74) (width 0.8) (layer B.Cu) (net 5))
 (segment (start 96.52 78.74) (end 104.14 78.74) (width 0.8) (layer B.Cu) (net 5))
 (segment (start 106.68 81.28) (end 106.68 83.82) (width 0.8) (layer B.Cu) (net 5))
 (segment (start 96.272058 78.74) (end 103.416 78.74) (width 0.8) (layer F.Cu) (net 5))
 (segment (start 103.416 78.74) (end 106.68 82.004) (width 0.8) (layer F.Cu) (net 5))
 (segment (start 106.68 82.004) (end 106.68 83.82) (width 0.8) (layer F.Cu) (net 5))
 (segment (start 81.540022 64.007964) (end 96.272058 78.74) (width 0.8) (layer F.Cu) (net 5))
 (segment (start 81.28 40.64) (end 83.82 40.64) (width 0.8) (layer F.Cu) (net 5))
 (segment (start 78.74 38.1) (end 81.28 40.64) (width 0.8) (layer F.Cu) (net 5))
 (segment (start 78.74 35.56) (end 78.74 38.1) (width 0.8) (layer F.Cu) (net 5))
 (segment (start 81.28 33.02) (end 78.74 35.56) (width 0.8) (layer F.Cu) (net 5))
 (segment (start 86.36 33.02) (end 81.28 33.02) (width 0.8) (layer F.Cu) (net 5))
 (segment (start 91.44 27.94) (end 86.36 33.02) (width 0.8) (layer F.Cu) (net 5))
 (segment (start 124.46 27.94) (end 91.44 27.94) (width 0.8) (layer F.Cu) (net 5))
 (segment (start 132.08 35.56) (end 124.46 27.94) (width 0.8) (layer F.Cu) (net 5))
 (segment (start 132.08 53.34) (end 132.08 35.56) (width 0.8) (layer F.Cu) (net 5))
 (segment (start 93.256 53.34) (end 93.98 54.064) (width 0.8) (layer F.Cu) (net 5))
 (segment (start 81.540022 64.007964) (end 81.540022 56.329892) (width 0.8) (layer F.Cu) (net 5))
 (segment (start 81.540022 56.329892) (end 84.529914 53.34) (width 0.8) (layer F.Cu) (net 5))
 (segment (start 84.529914 53.34) (end 93.256 53.34) (width 0.8) (layer F.Cu) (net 5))
 (segment (start 93.98 54.064) (end 93.98 55.88) (width 0.8) (layer F.Cu) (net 5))
 (segment (start 88.176 43.18) (end 88.176 48.26) (width 0.8) (layer F.Cu) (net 5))
 (segment (start 89.992 50.076) (end 88.176 48.26) (width 0.8) (layer F.Cu) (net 5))
 (segment (start 89.992 50.076) (end 93.98 54.064) (width 0.8) (layer F.Cu) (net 5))
 (segment (start 83.82 40.64) (end 85.636 40.64) (width 0.8) (layer F.Cu) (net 5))
 (segment (start 85.636 40.64) (end 88.176 43.18) (width 0.8) (layer F.Cu) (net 5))
 (segment (start 88.639979 48.723979) (end 93.256 53.34) (width 0.8) (layer B.Cu) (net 5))
 (segment (start 93.256 53.34) (end 93.98 54.064) (width 0.8) (layer B.Cu) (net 5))
 (segment (start 93.98 55.88) (end 93.98 54.064) (width 0.8) (layer B.Cu) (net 5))
 (segment (start 93.98 54.064) (end 93.779999 53.863999) (width 0.8) (layer B.Cu) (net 5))
 (segment (start 83.82 40.64) (end 85.636 40.64) (width 0.8) (layer B.Cu) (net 5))
 (segment (start 88.639979 43.643979) (end 88.639979 48.723979) (width 0.8) (layer B.Cu) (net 5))
 (segment (start 85.636 40.64) (end 88.639979 43.643979) (width 0.8) (layer B.Cu) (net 5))
 (segment (start 78.74 35.56) (end 78.74 37.376) (width 0.8) (layer B.Cu) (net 5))
 (segment (start 82.004 40.64) (end 83.82 40.64) (width 0.8) (layer B.Cu) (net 5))
 (segment (start 78.74 37.376) (end 82.004 40.64) (width 0.8) (layer B.Cu) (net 5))
 (segment (start 81.28 33.02) (end 78.74 35.56) (width 0.8) (layer B.Cu) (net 5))
 (segment (start 86.112058 33.02) (end 81.28 33.02) (width 0.8) (layer B.Cu) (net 5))
 (segment (start 124.46 27.94) (end 91.192058 27.94) (width 0.8) (layer B.Cu) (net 5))
 (segment (start 91.192058 27.94) (end 86.112058 33.02) (width 0.8) (layer B.Cu) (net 5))
 (segment (start 132.08 35.56) (end 124.46 27.94) (width 0.8) (layer B.Cu) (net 5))
 (segment (start 132.08 53.34) (end 132.08 35.56) (width 0.8) (layer B.Cu) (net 5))
 (segment (start 132.08 53.34) (end 132.08 51.524) (width 0.8) (layer B.Cu) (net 5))
 (segment (start 96.52 104.14) (end 93.732058 104.14) (width 0.8) (layer B.Cu) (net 7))
 (segment (start 93.732058 104.14) (end 83.82 94.227942) (width 0.8) (layer B.Cu) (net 7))
 (segment (start 83.82 94.227942) (end 83.82 86.36) (width 0.8) (layer B.Cu) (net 7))
 (segment (start 83.82 86.36) (end 83.82 83.82) (width 0.8) (layer B.Cu) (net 7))
 (segment (start 83.82 86.36) (end 83.82 83.82) (width 0.8) (layer F.Cu) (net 7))
 (segment (start 96.52 104.14) (end 93.732058 104.14) (width 0.8) (layer F.Cu) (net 7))
 (segment (start 93.732058 104.14) (end 83.82 94.227942) (width 0.8) (layer F.Cu) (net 7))
 (segment (start 83.82 94.227942) (end 83.82 86.36) (width 0.8) (layer F.Cu) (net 7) (status 20))
 (segment (start 99.06 104.14) (end 99.06 105.956) (width 0.8) (layer B.Cu) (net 8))
 (segment (start 86.36 82.004) (end 86.36 83.82) (width 0.8) (layer B.Cu) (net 8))
 (segment (start 99.06 105.956) (end 98.85999 106.15601) (width 0.8) (layer B.Cu) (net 8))
 (segment (start 98.85999 106.15601) (end 93.768155 106.15601) (width 0.8) (layer B.Cu) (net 8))
 (segment (start 93.768155 106.15601) (end 81.956399 94.344254) (width 0.8) (layer B.Cu) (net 8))
 (segment (start 81.956399 80.603601) (end 84.959601 80.603601) (width 0.8) (layer B.Cu) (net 8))
 (segment (start 81.956399 94.344254) (end 81.956399 80.603601) (width 0.8) (layer B.Cu) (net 8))
 (segment (start 84.959601 80.603601) (end 86.36 82.004) (width 0.8) (layer B.Cu) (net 8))
 (segment (start 99.06 104.14) (end 99.06 106.68) (width 0.8) (layer F.Cu) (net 8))
 (segment (start 99.06 106.68) (end 93.98 106.68) (width 0.8) (layer F.Cu) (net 8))
 (segment (start 93.98 106.68) (end 81.28 93.98) (width 0.8) (layer F.Cu) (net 8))
 (segment (start 81.28 93.98) (end 81.28 78.74) (width 0.8) (layer F.Cu) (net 8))
 (segment (start 81.28 78.74) (end 86.36 78.74) (width 0.8) (layer F.Cu) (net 8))
 (segment (start 86.36 78.74) (end 86.36 83.82) (width 0.8) (layer F.Cu) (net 8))
 (segment (start 78.479978 66.503978) (end 79.040065 66.503978) (width 0.8) (layer B.Cu) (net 12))
 (segment (start 79.040065 66.503978) (end 93.816087 81.28) (width 0.8) (layer B.Cu) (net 12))
 (segment (start 93.816087 81.28) (end 94.227942 81.28) (width 0.8) (layer B.Cu) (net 12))
 (segment (start 94.227942 81.28) (end 96.52 83.572058) (width 0.8) (layer B.Cu) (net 12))
 (segment (start 96.52 83.572058) (end 96.52 83.82) (width 0.8) (layer B.Cu) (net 12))
 (segment (start 83.82 43.18) (end 82.55 43.18) (width 0.8) (layer F.Cu) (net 12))
 (segment (start 78.74 46.99) (end 78.740001 65.16777) (width 0.8) (layer F.Cu) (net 12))
 (segment (start 82.55 43.18) (end 78.74 46.99) (width 0.8) (layer F.Cu) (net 12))
 (segment (start 78.740001 65.16777) (end 96.52 82.947769) (width 0.8) (layer F.Cu) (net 12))
 (segment (start 96.52 82.947769) (end 96.52 83.82) (width 0.8) (layer F.Cu) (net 12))
 (segment (start 78.479978 66.503978) (end 78.479978 46.704022) (width 0.8) (layer B.Cu) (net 12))
 (segment (start 78.479978 46.704022) (end 82.004 43.18) (width 0.8) (layer B.Cu) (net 12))
 (segment (start 82.004 43.18) (end 83.82 43.18) (width 0.8) (layer B.Cu) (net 12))
 (segment (start 79.87999 65.36399) (end 80.851932 65.36399) (width 0.8) (layer B.Cu) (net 13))
 (segment (start 80.851932 65.36399) (end 99.06 83.572058) (width 0.8) (layer B.Cu) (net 13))
 (segment (start 99.06 83.572058) (end 99.06 83.82) (width 0.8) (layer B.Cu) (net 13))
 (segment (start 80.140011 64.587867) (end 99.06 83.507856) (width 0.8) (layer F.Cu) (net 13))
 (segment (start 99.06 83.507856) (end 99.06 83.82) (width 0.8) (layer F.Cu) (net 13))
 (segment (start 83.82 47.3836) (end 80.140011 51.063589) (width 0.8) (layer F.Cu) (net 13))
 (segment (start 80.140011 51.063589) (end 80.140011 64.587867) (width 0.8) (layer F.Cu) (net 13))
 (segment (start 83.82 45.72) (end 83.82 47.3836) (width 0.8) (layer F.Cu) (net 13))
 (segment (start 83.82 47.3836) (end 83.82 45.72) (width 0.8) (layer B.Cu) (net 13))
 (segment (start 79.87999 65.36399) (end 79.87999 51.32361) (width 0.8) (layer B.Cu) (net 13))
 (segment (start 79.87999 51.32361) (end 83.82 47.3836) (width 0.8) (layer B.Cu) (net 13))
 (segment (start 119.38 63.5) (end 119.38 81.527942) (width 0.8) (layer F.Cu) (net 19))
 (segment (start 101.6 88.9) (end 96.52 93.98) (width 0.8) (layer F.Cu) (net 19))
 (segment (start 119.38 81.527942) (end 112.007942 88.9) (width 0.8) (layer F.Cu) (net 19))
 (segment (start 112.007942 88.9) (end 101.6 88.9) (width 0.8) (layer F.Cu) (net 19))
 (segment (start 96.52 93.98) (end 96.52 96.52) (width 0.8) (layer F.Cu) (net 19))
 (segment (start 96.52 96.52) (end 96.52 94.704) (width 0.8) (layer B.Cu) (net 19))
 (segment (start 96.52 94.704) (end 102.84799 88.37601) (width 0.8) (layer B.Cu) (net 19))
 (segment (start 102.84799 88.37601) (end 112.531932 88.37601) (width 0.8) (layer B.Cu) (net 19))
 (segment (start 112.531932 88.37601) (end 119.38 81.527942) (width 0.8) (layer B.Cu) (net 19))
 (segment (start 119.38 81.527942) (end 119.38 65.316) (width 0.8) (layer B.Cu) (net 19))
 (segment (start 119.38 65.316) (end 119.38 63.5) (width 0.8) (layer B.Cu) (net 19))
 (segment (start 88.9 63.5) (end 88.9 59.559602) (width 0.8) (layer F.Cu) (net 30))
 (segment (start 88.9 59.559602) (end 91.44 57.019602) (width 0.8) (layer F.Cu) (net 30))
 (segment (start 91.44 57.019602) (end 91.44 55.88) (width 0.8) (layer F.Cu) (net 30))
 (segment (start 91.44 55.88) (end 91.44 57.696) (width 0.8) (layer B.Cu) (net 30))
 (segment (start 91.44 57.696) (end 88.9 60.236) (width 0.8) (layer B.Cu) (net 30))
 (segment (start 88.9 60.236) (end 88.9 63.5) (width 0.8) (layer B.Cu) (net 30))
 (segment (start 86.36 63.5) (end 86.36 56.7564) (width 0.8) (layer F.Cu) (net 31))
 (segment (start 87.2364 55.88) (end 88.9 55.88) (width 0.8) (layer F.Cu) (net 31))
 (segment (start 86.36 56.7564) (end 87.2364 55.88) (width 0.8) (layer F.Cu) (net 31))
 (segment (start 86.36 58.5724) (end 86.36 61.684) (width 0.8) (layer B.Cu) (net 31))
 (segment (start 88.9 56.0324) (end 86.36 58.5724) (width 0.8) (layer B.Cu) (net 31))
 (segment (start 88.9 55.88) (end 88.9 56.0324) (width 0.8) (layer B.Cu) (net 31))
 (segment (start 86.36 61.684) (end 86.36 63.5) (width 0.8) (layer B.Cu) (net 31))
 (segment (start 95.25 48.26) (end 97.01911 48.26) (width 0.8) (layer F.Cu) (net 33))
 (segment (start 97.01911 48.26) (end 99.06 46.21911) (width 0.8) (layer F.Cu) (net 33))
 (segment (start 99.06 46.21911) (end 99.06 45.72) (width 0.8) (layer F.Cu) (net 33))
 (segment (start 86.36 39.37) (end 95.25 48.26) (width 0.8) (layer F.Cu) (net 33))
 (segment (start 86.36 38.1) (end 86.36 39.37) (width 0.8) (layer F.Cu) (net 33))
 (segment (start 83.82 38.1) (end 86.36 38.1) (width 0.8) (layer F.Cu) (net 33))
 (segment (start 97.01911 48.26) (end 96.085197 48.26) (width 0.8) (layer B.Cu) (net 33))
 (segment (start 96.085197 48.26) (end 85.925197 38.1) (width 0.8) (layer B.Cu) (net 33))
 (segment (start 85.925197 38.1) (end 85.636 38.1) (width 0.8) (layer B.Cu) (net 33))
 (segment (start 85.636 38.1) (end 83.82 38.1) (width 0.8) (layer B.Cu) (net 33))
 (segment (start 99.06 45.72) (end 99.06 46.21911) (width 0.8) (layer B.Cu) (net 33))
 (segment (start 99.06 46.21911) (end 97.01911 48.26) (width 0.8) (layer B.Cu) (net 33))
 (segment (start 96.52 55.88) (end 107.17911 55.88) (width 0.8) (layer F.Cu) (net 34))
 (segment (start 107.17911 55.88) (end 116.84 46.21911) (width 0.8) (layer F.Cu) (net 34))
 (segment (start 116.84 46.21911) (end 116.84 45.72) (width 0.8) (layer F.Cu) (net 34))
 (segment (start 116.84 45.72) (end 116.84 46.21911) (width 0.8) (layer B.Cu) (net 34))
 (segment (start 116.84 46.21911) (end 107.17911 55.88) (width 0.8) (layer B.Cu) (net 34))
 (segment (start 107.17911 55.88) (end 98.1836 55.88) (width 0.8) (layer B.Cu) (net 34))
 (segment (start 98.1836 55.88) (end 96.52 55.88) (width 0.8) (layer B.Cu) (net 34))
 (segment (start 95.25 44.45) (end 95.25 33.02) (width 0.8) (layer F.Cu) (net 35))
 (segment (start 96.52 45.72) (end 95.25 44.45) (width 0.8) (layer F.Cu) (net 35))
 (segment (start 95.25 33.02) (end 95.25 44.45) (width 0.8) (layer B.Cu) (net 35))
 (segment (start 95.25 44.45) (end 96.52 45.72) (width 0.8) (layer B.Cu) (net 35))
 (segment (start 113.03 33.02) (end 113.03 44.45) (width 0.8) (layer F.Cu) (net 36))
 (segment (start 113.03 44.45) (end 114.3 45.72) (width 0.8) (layer F.Cu) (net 36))
 (segment (start 113.03 33.02) (end 113.03 44.45) (width 0.8) (layer B.Cu) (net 36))
 (segment (start 113.03 44.45) (end 114.3 45.72) (width 0.8) (layer B.Cu) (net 36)))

